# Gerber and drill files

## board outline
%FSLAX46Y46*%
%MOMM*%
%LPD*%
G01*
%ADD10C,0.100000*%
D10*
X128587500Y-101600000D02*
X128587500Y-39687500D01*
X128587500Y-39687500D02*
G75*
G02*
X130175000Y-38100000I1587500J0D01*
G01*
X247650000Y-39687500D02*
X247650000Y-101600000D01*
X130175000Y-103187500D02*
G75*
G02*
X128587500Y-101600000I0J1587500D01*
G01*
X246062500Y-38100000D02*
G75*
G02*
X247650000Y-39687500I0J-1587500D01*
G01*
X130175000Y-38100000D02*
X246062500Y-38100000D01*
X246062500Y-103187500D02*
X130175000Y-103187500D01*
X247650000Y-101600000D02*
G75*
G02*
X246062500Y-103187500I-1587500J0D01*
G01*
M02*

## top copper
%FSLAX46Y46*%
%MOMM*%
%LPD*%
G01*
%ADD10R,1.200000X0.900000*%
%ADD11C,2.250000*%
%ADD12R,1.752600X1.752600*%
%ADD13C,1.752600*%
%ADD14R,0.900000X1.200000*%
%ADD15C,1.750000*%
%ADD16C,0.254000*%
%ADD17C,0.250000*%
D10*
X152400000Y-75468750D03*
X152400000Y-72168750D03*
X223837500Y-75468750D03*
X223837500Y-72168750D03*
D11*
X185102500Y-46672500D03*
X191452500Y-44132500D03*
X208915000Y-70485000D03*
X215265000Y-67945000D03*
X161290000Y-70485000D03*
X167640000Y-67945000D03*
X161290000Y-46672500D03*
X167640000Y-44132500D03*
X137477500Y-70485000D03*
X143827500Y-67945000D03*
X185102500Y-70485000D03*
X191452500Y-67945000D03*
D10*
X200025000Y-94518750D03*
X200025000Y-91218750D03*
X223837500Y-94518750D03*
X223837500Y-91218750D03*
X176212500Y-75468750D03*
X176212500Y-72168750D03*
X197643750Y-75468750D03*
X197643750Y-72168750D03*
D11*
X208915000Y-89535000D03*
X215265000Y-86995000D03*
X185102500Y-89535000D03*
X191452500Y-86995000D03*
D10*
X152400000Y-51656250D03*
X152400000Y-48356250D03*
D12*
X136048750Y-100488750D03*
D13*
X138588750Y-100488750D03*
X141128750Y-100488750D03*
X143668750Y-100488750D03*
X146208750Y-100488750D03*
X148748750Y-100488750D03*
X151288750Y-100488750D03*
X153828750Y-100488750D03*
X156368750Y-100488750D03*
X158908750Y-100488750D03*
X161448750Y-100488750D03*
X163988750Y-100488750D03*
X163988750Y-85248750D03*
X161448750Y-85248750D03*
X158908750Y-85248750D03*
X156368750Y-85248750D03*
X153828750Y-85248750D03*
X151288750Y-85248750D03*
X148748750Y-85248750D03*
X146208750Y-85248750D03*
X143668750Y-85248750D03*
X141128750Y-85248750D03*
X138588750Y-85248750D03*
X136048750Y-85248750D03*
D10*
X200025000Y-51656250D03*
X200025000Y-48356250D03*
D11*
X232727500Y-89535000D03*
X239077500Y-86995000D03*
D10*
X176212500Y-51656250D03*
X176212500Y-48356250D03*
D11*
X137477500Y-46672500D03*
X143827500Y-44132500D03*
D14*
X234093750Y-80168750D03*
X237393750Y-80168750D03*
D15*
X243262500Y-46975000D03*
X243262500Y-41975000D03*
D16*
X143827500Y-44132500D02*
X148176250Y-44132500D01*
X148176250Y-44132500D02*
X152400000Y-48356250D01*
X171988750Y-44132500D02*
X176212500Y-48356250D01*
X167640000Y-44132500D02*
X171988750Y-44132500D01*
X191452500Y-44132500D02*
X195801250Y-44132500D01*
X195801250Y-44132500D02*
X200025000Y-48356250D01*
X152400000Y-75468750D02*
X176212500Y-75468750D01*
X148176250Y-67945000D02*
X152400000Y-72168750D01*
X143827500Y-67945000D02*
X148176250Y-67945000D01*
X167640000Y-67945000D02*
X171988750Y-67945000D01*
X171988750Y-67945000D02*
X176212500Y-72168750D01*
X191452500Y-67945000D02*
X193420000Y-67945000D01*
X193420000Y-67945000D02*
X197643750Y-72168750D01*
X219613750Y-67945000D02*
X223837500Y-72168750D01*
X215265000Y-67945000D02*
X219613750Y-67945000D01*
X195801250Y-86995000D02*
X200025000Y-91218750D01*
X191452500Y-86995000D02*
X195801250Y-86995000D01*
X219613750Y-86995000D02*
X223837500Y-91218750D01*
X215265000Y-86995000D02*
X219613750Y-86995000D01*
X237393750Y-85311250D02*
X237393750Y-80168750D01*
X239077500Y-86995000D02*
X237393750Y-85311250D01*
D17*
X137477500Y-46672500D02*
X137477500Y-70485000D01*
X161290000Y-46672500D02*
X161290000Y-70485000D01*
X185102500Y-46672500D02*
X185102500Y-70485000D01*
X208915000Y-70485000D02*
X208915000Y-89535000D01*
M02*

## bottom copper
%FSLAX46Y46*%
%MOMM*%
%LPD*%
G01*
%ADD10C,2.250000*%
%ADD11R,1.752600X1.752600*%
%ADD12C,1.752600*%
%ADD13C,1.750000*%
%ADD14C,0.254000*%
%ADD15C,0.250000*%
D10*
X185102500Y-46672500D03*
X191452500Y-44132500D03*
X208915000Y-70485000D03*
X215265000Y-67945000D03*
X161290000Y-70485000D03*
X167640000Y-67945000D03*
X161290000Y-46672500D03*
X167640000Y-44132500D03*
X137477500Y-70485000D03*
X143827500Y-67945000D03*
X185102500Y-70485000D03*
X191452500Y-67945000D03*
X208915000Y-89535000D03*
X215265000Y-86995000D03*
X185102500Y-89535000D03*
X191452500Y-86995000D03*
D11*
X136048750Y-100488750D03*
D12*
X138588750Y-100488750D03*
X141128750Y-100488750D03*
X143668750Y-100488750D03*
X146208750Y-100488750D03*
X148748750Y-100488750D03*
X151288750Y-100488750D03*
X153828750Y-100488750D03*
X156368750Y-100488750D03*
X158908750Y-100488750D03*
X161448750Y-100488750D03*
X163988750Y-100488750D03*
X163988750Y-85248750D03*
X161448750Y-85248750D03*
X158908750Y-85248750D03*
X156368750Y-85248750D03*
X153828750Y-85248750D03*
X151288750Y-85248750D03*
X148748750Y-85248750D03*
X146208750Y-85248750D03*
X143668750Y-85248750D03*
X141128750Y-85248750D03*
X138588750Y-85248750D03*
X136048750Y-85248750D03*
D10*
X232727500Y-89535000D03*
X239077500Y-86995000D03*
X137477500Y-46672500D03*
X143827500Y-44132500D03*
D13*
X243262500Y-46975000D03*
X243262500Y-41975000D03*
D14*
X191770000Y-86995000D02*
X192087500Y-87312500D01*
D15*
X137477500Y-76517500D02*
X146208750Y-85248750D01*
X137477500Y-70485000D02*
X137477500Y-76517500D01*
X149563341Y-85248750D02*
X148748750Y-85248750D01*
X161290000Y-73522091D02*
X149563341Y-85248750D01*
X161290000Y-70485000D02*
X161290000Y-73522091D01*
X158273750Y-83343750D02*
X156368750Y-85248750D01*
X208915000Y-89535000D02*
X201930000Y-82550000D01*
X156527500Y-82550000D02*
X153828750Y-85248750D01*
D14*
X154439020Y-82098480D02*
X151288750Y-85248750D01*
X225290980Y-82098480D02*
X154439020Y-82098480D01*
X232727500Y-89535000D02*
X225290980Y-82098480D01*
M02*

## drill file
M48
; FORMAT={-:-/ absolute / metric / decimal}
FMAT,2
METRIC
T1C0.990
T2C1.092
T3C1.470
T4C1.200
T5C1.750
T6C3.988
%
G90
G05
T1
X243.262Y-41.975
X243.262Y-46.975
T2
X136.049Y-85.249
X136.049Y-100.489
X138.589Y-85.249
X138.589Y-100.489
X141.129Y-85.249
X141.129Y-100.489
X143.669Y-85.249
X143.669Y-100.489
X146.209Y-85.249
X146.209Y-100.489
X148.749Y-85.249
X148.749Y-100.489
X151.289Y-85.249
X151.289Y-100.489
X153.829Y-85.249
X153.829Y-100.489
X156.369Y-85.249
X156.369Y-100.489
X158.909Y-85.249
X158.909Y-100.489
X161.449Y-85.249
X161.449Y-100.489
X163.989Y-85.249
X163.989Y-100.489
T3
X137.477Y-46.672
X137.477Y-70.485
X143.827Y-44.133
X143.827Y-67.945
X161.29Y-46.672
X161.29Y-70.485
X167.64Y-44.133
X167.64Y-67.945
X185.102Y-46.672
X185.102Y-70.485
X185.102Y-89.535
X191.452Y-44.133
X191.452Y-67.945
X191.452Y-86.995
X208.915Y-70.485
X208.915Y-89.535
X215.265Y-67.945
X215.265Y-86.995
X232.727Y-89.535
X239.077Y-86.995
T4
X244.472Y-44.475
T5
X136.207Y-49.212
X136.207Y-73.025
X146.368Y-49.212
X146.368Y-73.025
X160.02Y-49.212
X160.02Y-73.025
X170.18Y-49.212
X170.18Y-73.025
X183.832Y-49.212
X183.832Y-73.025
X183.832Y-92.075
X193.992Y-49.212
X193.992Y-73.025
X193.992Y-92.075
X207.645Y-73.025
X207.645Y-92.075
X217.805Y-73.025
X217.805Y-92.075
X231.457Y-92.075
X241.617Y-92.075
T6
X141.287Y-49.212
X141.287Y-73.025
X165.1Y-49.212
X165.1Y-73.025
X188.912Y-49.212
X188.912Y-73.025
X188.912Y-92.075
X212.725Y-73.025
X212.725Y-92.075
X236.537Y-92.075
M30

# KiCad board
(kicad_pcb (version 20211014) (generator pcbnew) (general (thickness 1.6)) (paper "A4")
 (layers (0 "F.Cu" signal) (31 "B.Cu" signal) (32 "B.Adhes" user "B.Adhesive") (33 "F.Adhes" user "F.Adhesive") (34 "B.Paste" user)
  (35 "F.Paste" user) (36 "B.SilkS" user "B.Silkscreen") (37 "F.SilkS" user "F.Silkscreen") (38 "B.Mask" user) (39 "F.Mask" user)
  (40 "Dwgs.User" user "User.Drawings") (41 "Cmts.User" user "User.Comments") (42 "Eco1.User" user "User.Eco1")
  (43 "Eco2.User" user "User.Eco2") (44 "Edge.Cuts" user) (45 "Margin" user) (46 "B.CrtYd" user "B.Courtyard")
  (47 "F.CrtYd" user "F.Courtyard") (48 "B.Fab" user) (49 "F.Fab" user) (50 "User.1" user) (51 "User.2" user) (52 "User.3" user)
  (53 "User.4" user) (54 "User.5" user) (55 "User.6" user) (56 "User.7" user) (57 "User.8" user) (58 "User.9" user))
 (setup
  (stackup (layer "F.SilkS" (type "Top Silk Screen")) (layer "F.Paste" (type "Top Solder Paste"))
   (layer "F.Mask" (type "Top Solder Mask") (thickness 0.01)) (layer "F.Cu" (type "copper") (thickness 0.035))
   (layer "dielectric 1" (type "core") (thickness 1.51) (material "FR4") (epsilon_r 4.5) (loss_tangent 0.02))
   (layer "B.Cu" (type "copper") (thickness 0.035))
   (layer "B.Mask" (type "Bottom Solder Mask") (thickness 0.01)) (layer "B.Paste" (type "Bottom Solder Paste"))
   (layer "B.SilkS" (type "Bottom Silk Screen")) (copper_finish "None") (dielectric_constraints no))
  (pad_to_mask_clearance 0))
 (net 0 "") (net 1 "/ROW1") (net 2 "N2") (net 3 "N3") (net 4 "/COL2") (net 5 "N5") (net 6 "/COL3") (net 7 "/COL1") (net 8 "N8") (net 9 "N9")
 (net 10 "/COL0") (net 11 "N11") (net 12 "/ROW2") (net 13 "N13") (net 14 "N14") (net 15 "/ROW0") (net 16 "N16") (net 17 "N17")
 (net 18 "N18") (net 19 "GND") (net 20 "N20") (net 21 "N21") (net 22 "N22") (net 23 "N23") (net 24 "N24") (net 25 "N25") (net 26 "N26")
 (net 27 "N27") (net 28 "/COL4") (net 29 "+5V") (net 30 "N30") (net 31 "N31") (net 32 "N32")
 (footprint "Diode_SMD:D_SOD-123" (layer "F.Cu") (at 152.4 73.81875 90)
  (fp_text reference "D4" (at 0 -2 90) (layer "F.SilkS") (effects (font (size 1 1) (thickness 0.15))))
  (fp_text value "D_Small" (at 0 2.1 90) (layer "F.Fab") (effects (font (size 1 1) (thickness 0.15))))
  (pad "1" smd rect (at -1.65 0 90) (size 0.9 1.2) (layers "F.Cu" "F.Paste" "F.Mask") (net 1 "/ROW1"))
  (pad "2" smd rect (at 1.65 0 90) (size 0.9 1.2) (layers "F.Cu" "F.Paste" "F.Mask") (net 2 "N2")))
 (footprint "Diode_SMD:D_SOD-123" (layer "F.Cu") (at 223.8375 73.81875 90)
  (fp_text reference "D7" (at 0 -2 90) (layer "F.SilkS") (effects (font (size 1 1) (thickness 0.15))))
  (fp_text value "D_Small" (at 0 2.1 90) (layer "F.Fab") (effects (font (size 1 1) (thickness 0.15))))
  (pad "1" smd rect (at -1.65 0 90) (size 0.9 1.2) (layers "F.Cu" "F.Paste" "F.Mask") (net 1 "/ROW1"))
  (pad "2" smd rect (at 1.65 0 90) (size 0.9 1.2) (layers "F.Cu" "F.Paste" "F.Mask") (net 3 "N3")))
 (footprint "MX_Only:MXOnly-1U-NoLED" (layer "F.Cu") (at 188.9125 49.2125)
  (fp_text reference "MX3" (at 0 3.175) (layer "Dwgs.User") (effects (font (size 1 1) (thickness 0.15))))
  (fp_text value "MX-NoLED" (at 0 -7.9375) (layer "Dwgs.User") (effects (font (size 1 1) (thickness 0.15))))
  (pad "" np_thru_hole circle locked (at 0 0) (size 3.9878 3.9878) (drill 3.9878) (layers *.Cu *.Mask))
  (pad "" np_thru_hole circle locked (at -5.08 0 48.0996) (size 1.75 1.75) (drill 1.75) (layers *.Cu *.Mask))
  (pad "" np_thru_hole circle locked (at 5.08 0 48.0996) (size 1.75 1.75) (drill 1.75) (layers *.Cu *.Mask))
  (pad "1" thru_hole circle locked (at -3.81 -2.54) (size 2.25 2.25) (drill 1.47) (layers *.Cu "B.Mask") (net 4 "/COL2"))
  (pad "2" thru_hole circle locked (at 2.54 -5.08) (size 2.25 2.25) (drill 1.47) (layers *.Cu "B.Mask") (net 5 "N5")))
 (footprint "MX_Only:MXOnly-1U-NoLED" (layer "F.Cu") (at 212.725 73.025)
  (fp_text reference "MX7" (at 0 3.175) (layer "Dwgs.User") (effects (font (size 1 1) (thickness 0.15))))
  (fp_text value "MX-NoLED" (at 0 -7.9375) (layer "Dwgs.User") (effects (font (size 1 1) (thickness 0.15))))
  (pad "" np_thru_hole circle locked (at 5.08 0 48.0996) (size 1.75 1.75) (drill 1.75) (layers *.Cu *.Mask))
  (pad "" np_thru_hole circle locked (at 0 0) (size 3.9878 3.9878) (drill 3.9878) (layers *.Cu *.Mask))
  (pad "" np_thru_hole circle locked (at -5.08 0 48.0996) (size 1.75 1.75) (drill 1.75) (layers *.Cu *.Mask))
  (pad "1" thru_hole circle locked (at -3.81 -2.54) (size 2.25 2.25) (drill 1.47) (layers *.Cu "B.Mask") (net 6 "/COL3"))
  (pad "2" thru_hole circle locked (at 2.54 -5.08) (size 2.25 2.25) (drill 1.47) (layers *.Cu "B.Mask") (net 3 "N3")))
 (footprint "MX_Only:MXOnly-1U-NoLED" (layer "F.Cu") (at 165.1 73.025)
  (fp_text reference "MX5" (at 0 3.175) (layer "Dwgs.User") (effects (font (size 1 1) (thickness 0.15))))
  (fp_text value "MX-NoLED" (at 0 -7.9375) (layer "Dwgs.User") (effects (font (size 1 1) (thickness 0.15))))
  (pad "" np_thru_hole circle locked (at 5.08 0 48.0996) (size 1.75 1.75) (drill 1.75) (layers *.Cu *.Mask))
  (pad "" np_thru_hole circle locked (at -5.08 0 48.0996) (size 1.75 1.75) (drill 1.75) (layers *.Cu *.Mask))
  (pad "" np_thru_hole circle locked (at 0 0) (size 3.9878 3.9878) (drill 3.9878) (layers *.Cu *.Mask))
  (pad "1" thru_hole circle locked (at -3.81 -2.54) (size 2.25 2.25) (drill 1.47) (layers *.Cu "B.Mask") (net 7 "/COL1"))
  (pad "2" thru_hole circle locked (at 2.54 -5.08) (size 2.25 2.25) (drill 1.47) (layers *.Cu "B.Mask") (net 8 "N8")))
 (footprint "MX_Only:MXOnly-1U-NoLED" (layer "F.Cu") (at 165.1 49.2125)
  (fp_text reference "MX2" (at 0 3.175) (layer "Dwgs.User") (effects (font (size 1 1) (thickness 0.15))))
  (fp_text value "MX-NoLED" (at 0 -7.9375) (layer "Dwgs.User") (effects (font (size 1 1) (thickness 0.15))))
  (pad "" np_thru_hole circle locked (at 5.08 0 48.0996) (size 1.75 1.75) (drill 1.75) (layers *.Cu *.Mask))
  (pad "" np_thru_hole circle locked (at 0 0) (size 3.9878 3.9878) (drill 3.9878) (layers *.Cu *.Mask))
  (pad "" np_thru_hole circle locked (at -5.08 0 48.0996) (size 1.75 1.75) (drill 1.75) (layers *.Cu *.Mask))
  (pad "1" thru_hole circle locked (at -3.81 -2.54) (size 2.25 2.25) (drill 1.47) (layers *.Cu "B.Mask") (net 7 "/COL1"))
  (pad "2" thru_hole circle locked (at 2.54 -5.08) (size 2.25 2.25) (drill 1.47) (layers *.Cu "B.Mask") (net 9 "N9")))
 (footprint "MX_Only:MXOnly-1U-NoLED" (layer "F.Cu") (at 141.2875 73.025)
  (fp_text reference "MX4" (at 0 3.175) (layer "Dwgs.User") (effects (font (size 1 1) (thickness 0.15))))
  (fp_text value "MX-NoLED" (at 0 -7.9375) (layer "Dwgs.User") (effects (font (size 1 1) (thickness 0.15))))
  (pad "" np_thru_hole circle locked (at 0 0) (size 3.9878 3.9878) (drill 3.9878) (layers *.Cu *.Mask))
  (pad "" np_thru_hole circle locked (at -5.08 0 48.0996) (size 1.75 1.75) (drill 1.75) (layers *.Cu *.Mask))
  (pad "" np_thru_hole circle locked (at 5.08 0 48.0996) (size 1.75 1.75) (drill 1.75) (layers *.Cu *.Mask))
  (pad "1" thru_hole circle locked (at -3.81 -2.54) (size 2.25 2.25) (drill 1.47) (layers *.Cu "B.Mask") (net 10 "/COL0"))
  (pad "2" thru_hole circle locked (at 2.54 -5.08) (size 2.25 2.25) (drill 1.47) (layers *.Cu "B.Mask") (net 2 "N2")))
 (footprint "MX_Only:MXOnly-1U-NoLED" (layer "F.Cu") (at 188.9125 73.025)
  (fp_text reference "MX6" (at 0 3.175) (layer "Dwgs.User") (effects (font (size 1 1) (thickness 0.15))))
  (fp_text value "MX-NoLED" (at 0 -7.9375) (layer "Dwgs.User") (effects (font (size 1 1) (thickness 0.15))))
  (pad "" np_thru_hole circle locked (at -5.08 0 48.0996) (size 1.75 1.75) (drill 1.75) (layers *.Cu *.Mask))
  (pad "" np_thru_hole circle locked (at 5.08 0 48.0996) (size 1.75 1.75) (drill 1.75) (layers *.Cu *.Mask))
  (pad "" np_thru_hole circle locked (at 0 0) (size 3.9878 3.9878) (drill 3.9878) (layers *.Cu *.Mask))
  (pad "1" thru_hole circle locked (at -3.81 -2.54) (size 2.25 2.25) (drill 1.47) (layers *.Cu "B.Mask") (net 4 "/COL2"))
  (pad "2" thru_hole circle locked (at 2.54 -5.08) (size 2.25 2.25) (drill 1.47) (layers *.Cu "B.Mask") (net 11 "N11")))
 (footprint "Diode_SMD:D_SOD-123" (layer "F.Cu") (at 200.025 92.86875 90)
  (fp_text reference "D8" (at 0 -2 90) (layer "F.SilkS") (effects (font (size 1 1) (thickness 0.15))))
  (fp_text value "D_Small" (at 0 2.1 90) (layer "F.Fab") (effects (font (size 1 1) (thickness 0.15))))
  (pad "1" smd rect (at -1.65 0 90) (size 0.9 1.2) (layers "F.Cu" "F.Paste" "F.Mask") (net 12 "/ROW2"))
  (pad "2" smd rect (at 1.65 0 90) (size 0.9 1.2) (layers "F.Cu" "F.Paste" "F.Mask") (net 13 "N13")))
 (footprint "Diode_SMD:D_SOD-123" (layer "F.Cu") (at 223.8375 92.86875 90)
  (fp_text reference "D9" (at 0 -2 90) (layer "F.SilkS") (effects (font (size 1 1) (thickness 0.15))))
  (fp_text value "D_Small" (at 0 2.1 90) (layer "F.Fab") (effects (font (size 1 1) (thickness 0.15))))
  (pad "1" smd rect (at -1.65 0 90) (size 0.9 1.2) (layers "F.Cu" "F.Paste" "F.Mask") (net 12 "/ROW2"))
  (pad "2" smd rect (at 1.65 0 90) (size 0.9 1.2) (layers "F.Cu" "F.Paste" "F.Mask") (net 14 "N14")))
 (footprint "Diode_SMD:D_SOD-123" (layer "F.Cu") (at 176.2125 73.81875 90)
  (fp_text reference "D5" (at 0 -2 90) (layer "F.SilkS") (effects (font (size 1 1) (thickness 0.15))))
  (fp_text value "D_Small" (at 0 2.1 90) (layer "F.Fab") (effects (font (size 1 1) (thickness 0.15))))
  (pad "1" smd rect (at -1.65 0 90) (size 0.9 1.2) (layers "F.Cu" "F.Paste" "F.Mask") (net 1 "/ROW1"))
  (pad "2" smd rect (at 1.65 0 90) (size 0.9 1.2) (layers "F.Cu" "F.Paste" "F.Mask") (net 8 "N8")))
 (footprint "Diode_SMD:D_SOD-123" (layer "F.Cu") (at 197.64375 73.81875 90)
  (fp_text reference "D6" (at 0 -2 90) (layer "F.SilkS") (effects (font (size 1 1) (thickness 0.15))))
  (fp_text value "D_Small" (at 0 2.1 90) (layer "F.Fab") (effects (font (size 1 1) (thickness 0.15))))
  (pad "1" smd rect (at -1.65 0 90) (size 0.9 1.2) (layers "F.Cu" "F.Paste" "F.Mask") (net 1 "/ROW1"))
  (pad "2" smd rect (at 1.65 0 90) (size 0.9 1.2) (layers "F.Cu" "F.Paste" "F.Mask") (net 11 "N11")))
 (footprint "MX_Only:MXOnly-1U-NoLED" (layer "F.Cu") (at 212.725 92.075)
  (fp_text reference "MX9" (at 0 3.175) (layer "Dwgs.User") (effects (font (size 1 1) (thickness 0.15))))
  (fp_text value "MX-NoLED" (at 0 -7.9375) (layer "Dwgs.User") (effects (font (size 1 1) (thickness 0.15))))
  (pad "" np_thru_hole circle locked (at 0 0) (size 3.9878 3.9878) (drill 3.9878) (layers *.Cu *.Mask))
  (pad "" np_thru_hole circle locked (at 5.08 0 48.0996) (size 1.75 1.75) (drill 1.75) (layers *.Cu *.Mask))
  (pad "" np_thru_hole circle locked (at -5.08 0 48.0996) (size 1.75 1.75) (drill 1.75) (layers *.Cu *.Mask))
  (pad "1" thru_hole circle locked (at -3.81 -2.54) (size 2.25 2.25) (drill 1.47) (layers *.Cu "B.Mask") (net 6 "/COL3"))
  (pad "2" thru_hole circle locked (at 2.54 -5.08) (size 2.25 2.25) (drill 1.47) (layers *.Cu "B.Mask") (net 14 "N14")))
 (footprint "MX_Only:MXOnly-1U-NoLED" (layer "F.Cu") (at 188.9125 92.075)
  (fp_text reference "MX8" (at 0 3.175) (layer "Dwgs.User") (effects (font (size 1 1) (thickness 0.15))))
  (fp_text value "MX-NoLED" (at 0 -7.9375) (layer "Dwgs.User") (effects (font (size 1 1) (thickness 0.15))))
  (pad "" np_thru_hole circle locked (at 5.08 0 48.0996) (size 1.75 1.75) (drill 1.75) (layers *.Cu *.Mask))
  (pad "" np_thru_hole circle locked (at 0 0) (size 3.9878 3.9878) (drill 3.9878) (layers *.Cu *.Mask))
  (pad "" np_thru_hole circle locked (at -5.08 0 48.0996) (size 1.75 1.75) (drill 1.75) (layers *.Cu *.Mask))
  (pad "1" thru_hole circle locked (at -3.81 -2.54) (size 2.25 2.25) (drill 1.47) (layers *.Cu "B.Mask") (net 4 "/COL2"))
  (pad "2" thru_hole circle locked (at 2.54 -5.08) (size 2.25 2.25) (drill 1.47) (layers *.Cu "B.Mask") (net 13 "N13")))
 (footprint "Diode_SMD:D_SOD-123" (layer "F.Cu") (at 152.4 50.00625 90)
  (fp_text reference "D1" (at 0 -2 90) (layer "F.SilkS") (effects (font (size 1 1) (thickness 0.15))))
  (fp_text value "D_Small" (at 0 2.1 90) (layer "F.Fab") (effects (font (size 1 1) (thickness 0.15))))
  (pad "1" smd rect (at -1.65 0 90) (size 0.9 1.2) (layers "F.Cu" "F.Paste" "F.Mask") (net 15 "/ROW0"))
  (pad "2" smd rect (at 1.65 0 90) (size 0.9 1.2) (layers "F.Cu" "F.Paste" "F.Mask") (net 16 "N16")))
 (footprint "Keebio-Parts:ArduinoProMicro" (layer "F.Cu") (at 150.01875 92.86875)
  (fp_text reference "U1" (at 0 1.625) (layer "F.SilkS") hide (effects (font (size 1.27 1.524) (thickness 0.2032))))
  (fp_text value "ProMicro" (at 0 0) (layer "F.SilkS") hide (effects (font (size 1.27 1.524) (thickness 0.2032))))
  (pad "1" thru_hole rect locked (at -13.97 7.62) (size 1.7526 1.7526) (drill 1.0922) (layers *.Cu *.SilkS *.Mask) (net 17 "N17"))
  (pad "2" thru_hole circle locked (at -11.43 7.62) (size 1.7526 1.7526) (drill 1.0922) (layers *.Cu *.SilkS *.Mask) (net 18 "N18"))
  (pad "3" thru_hole circle locked (at -8.89 7.62) (size 1.7526 1.7526) (drill 1.0922) (layers *.Cu *.SilkS *.Mask) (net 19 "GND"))
  (pad "4" thru_hole circle locked (at -6.35 7.62) (size 1.7526 1.7526) (drill 1.0922) (layers *.Cu *.SilkS *.Mask) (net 19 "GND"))
  (pad "5" thru_hole circle locked (at -3.81 7.62) (size 1.7526 1.7526) (drill 1.0922) (layers *.Cu *.SilkS *.Mask) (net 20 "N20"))
  (pad "6" thru_hole circle locked (at -1.27 7.62) (size 1.7526 1.7526) (drill 1.0922) (layers *.Cu *.SilkS *.Mask) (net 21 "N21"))
  (pad "7" thru_hole circle locked (at 1.27 7.62) (size 1.7526 1.7526) (drill 1.0922) (layers *.Cu *.SilkS *.Mask) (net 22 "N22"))
  (pad "8" thru_hole circle locked (at 3.81 7.62) (size 1.7526 1.7526) (drill 1.0922) (layers *.Cu *.SilkS *.Mask) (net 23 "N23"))
  (pad "9" thru_hole circle locked (at 6.35 7.62) (size 1.7526 1.7526) (drill 1.0922) (layers *.Cu *.SilkS *.Mask) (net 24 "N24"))
  (pad "10" thru_hole circle locked (at 8.89 7.62) (size 1.7526 1.7526) (drill 1.0922) (layers *.Cu *.SilkS *.Mask) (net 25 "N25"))
  (pad "11" thru_hole circle locked (at 11.43 7.62) (size 1.7526 1.7526) (drill 1.0922) (layers *.Cu *.SilkS *.Mask) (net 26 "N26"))
  (pad "12" thru_hole circle locked (at 13.97 7.62) (size 1.7526 1.7526) (drill 1.0922) (layers *.Cu *.SilkS *.Mask) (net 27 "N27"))
  (pad "13" thru_hole circle locked (at 13.97 -7.62) (size 1.7526 1.7526) (drill 1.0922) (layers *.Cu *.SilkS *.Mask) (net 12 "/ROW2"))
  (pad "14" thru_hole circle locked (at 11.43 -7.62) (size 1.7526 1.7526) (drill 1.0922) (layers *.Cu *.SilkS *.Mask) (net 1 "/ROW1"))
  (pad "15" thru_hole circle locked (at 8.89 -7.62) (size 1.7526 1.7526) (drill 1.0922) (layers *.Cu *.SilkS *.Mask) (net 15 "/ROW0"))
  (pad "16" thru_hole circle locked (at 6.35 -7.62) (size 1.7526 1.7526) (drill 1.0922) (layers *.Cu *.SilkS *.Mask) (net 4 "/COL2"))
  (pad "17" thru_hole circle locked (at 3.81 -7.62) (size 1.7526 1.7526) (drill 1.0922) (layers *.Cu *.SilkS *.Mask) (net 6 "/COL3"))
  (pad "18" thru_hole circle locked (at 1.27 -7.62) (size 1.7526 1.7526) (drill 1.0922) (layers *.Cu *.SilkS *.Mask) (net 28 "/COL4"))
  (pad "19" thru_hole circle locked (at -1.27 -7.62) (size 1.7526 1.7526) (drill 1.0922) (layers *.Cu *.SilkS *.Mask) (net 7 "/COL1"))
  (pad "20" thru_hole circle locked (at -3.81 -7.62) (size 1.7526 1.7526) (drill 1.0922) (layers *.Cu *.SilkS *.Mask) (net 10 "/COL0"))
  (pad "21" thru_hole circle locked (at -6.35 -7.62) (size 1.7526 1.7526) (drill 1.0922) (layers *.Cu *.SilkS *.Mask) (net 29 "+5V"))
  (pad "22" thru_hole circle locked (at -8.89 -7.62) (size 1.7526 1.7526) (drill 1.0922) (layers *.Cu *.SilkS *.Mask) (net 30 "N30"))
  (pad "23" thru_hole circle locked (at -11.43 -7.62) (size 1.7526 1.7526) (drill 1.0922) (layers *.Cu *.SilkS *.Mask) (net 19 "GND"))
  (pad "24" thru_hole circle locked (at -13.97 -7.62) (size 1.7526 1.7526) (drill 1.0922) (layers *.Cu *.SilkS *.Mask) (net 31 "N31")))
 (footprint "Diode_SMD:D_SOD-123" (layer "F.Cu") (at 200.025 50.00625 90)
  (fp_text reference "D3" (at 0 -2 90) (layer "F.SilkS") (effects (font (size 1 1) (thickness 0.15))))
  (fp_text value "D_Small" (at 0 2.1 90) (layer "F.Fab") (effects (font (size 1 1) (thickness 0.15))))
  (pad "1" smd rect (at -1.65 0 90) (size 0.9 1.2) (layers "F.Cu" "F.Paste" "F.Mask") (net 15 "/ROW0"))
  (pad "2" smd rect (at 1.65 0 90) (size 0.9 1.2) (layers "F.Cu" "F.Paste" "F.Mask") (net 5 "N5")))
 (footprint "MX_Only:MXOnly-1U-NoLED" (layer "F.Cu") (at 236.5375 92.075)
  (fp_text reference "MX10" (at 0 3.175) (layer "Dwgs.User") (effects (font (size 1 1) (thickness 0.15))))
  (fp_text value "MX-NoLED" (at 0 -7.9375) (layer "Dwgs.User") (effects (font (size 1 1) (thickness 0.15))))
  (pad "" np_thru_hole circle locked (at 0 0) (size 3.9878 3.9878) (drill 3.9878) (layers *.Cu *.Mask))
  (pad "" np_thru_hole circle locked (at 5.08 0 48.0996) (size 1.75 1.75) (drill 1.75) (layers *.Cu *.Mask))
  (pad "" np_thru_hole circle locked (at -5.08 0 48.0996) (size 1.75 1.75) (drill 1.75) (layers *.Cu *.Mask))
  (pad "1" thru_hole circle locked (at -3.81 -2.54) (size 2.25 2.25) (drill 1.47) (layers *.Cu "B.Mask") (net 28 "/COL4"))
  (pad "2" thru_hole circle locked (at 2.54 -5.08) (size 2.25 2.25) (drill 1.47) (layers *.Cu "B.Mask") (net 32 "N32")))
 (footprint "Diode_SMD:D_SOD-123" (layer "F.Cu") (at 176.2125 50.00625 90)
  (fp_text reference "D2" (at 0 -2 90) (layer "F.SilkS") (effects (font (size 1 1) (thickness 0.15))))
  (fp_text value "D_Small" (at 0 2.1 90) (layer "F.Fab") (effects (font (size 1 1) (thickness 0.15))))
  (pad "1" smd rect (at -1.65 0 90) (size 0.9 1.2) (layers "F.Cu" "F.Paste" "F.Mask") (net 15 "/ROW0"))
  (pad "2" smd rect (at 1.65 0 90) (size 0.9 1.2) (layers "F.Cu" "F.Paste" "F.Mask") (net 9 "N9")))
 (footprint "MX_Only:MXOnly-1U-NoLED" (layer "F.Cu") (at 141.2875 49.2125)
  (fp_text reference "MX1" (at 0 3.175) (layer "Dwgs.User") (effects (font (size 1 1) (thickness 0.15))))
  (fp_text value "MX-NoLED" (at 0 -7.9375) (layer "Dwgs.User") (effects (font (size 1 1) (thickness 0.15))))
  (pad "" np_thru_hole circle locked (at 0 0) (size 3.9878 3.9878) (drill 3.9878) (layers *.Cu *.Mask))
  (pad "" np_thru_hole circle locked (at -5.08 0 48.0996) (size 1.75 1.75) (drill 1.75) (layers *.Cu *.Mask))
  (pad "" np_thru_hole circle locked (at 5.08 0 48.0996) (size 1.75 1.75) (drill 1.75) (layers *.Cu *.Mask))
  (pad "1" thru_hole circle locked (at -3.81 -2.54) (size 2.25 2.25) (drill 1.47) (layers *.Cu "B.Mask") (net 10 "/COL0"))
  (pad "2" thru_hole circle locked (at 2.54 -5.08) (size 2.25 2.25) (drill 1.47) (layers *.Cu "B.Mask") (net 16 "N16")))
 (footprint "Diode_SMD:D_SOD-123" (layer "F.Cu") (at 235.74375 80.16875)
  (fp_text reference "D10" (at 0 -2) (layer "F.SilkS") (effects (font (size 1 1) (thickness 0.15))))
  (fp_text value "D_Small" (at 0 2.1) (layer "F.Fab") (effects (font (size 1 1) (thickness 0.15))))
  (pad "1" smd rect (at -1.65 0) (size 0.9 1.2) (layers "F.Cu" "F.Paste" "F.Mask") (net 12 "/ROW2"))
  (pad "2" smd rect (at 1.65 0) (size 0.9 1.2) (layers "F.Cu" "F.Paste" "F.Mask") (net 32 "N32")))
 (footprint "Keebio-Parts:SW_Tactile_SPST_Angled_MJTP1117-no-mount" (layer "B.Cu") (at 243.2625 46.975 90)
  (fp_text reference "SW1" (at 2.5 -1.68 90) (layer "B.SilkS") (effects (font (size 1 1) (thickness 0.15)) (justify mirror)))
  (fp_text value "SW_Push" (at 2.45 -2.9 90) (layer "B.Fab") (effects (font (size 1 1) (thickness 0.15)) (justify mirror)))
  (pad "" np_thru_hole circle locked (at 2.5 1.21 90) (size 1.2 1.2) (drill 1.2) (layers *.Cu *.Mask))
  (pad "1" thru_hole circle locked (at 0 0 90) (size 1.75 1.75) (drill 0.99) (layers *.Cu *.Mask) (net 30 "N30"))
  (pad "2" thru_hole circle locked (at 5 0 90) (size 1.75 1.75) (drill 0.99) (layers *.Cu *.Mask) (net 19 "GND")))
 (gr_line (start 128.5875 101.6) (end 128.5875 39.6875) (layer "Edge.Cuts") (width 0.1))
 (gr_arc (start 128.5875 39.6875) (mid 129.052468 38.564968) (end 130.175 38.1) (layer "Edge.Cuts") (width 0.1))
 (gr_line (start 247.65 39.6875) (end 247.65 101.6) (layer "Edge.Cuts") (width 0.1))
 (gr_arc (start 130.175 103.1875) (mid 129.052468 102.722532) (end 128.5875 101.6) (layer "Edge.Cuts") (width 0.1))
 (gr_arc (start 246.0625 38.1) (mid 247.185032 38.564968) (end 247.65 39.6875) (layer "Edge.Cuts") (width 0.1))
 (gr_line (start 130.175 38.1) (end 246.0625 38.1) (layer "Edge.Cuts") (width 0.1))
 (gr_line (start 246.0625 103.1875) (end 130.175 103.1875) (layer "Edge.Cuts") (width 0.1))
 (gr_arc (start 247.65 101.6) (mid 247.185032 102.722532) (end 246.0625 103.1875) (layer "Edge.Cuts") (width 0.1))
 (segment (start 143.8275 44.1325) (end 148.17625 44.1325) (width 0.254) (layer "F.Cu") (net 16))
 (segment (start 148.17625 44.1325) (end 152.4 48.35625) (width 0.254) (layer "F.Cu") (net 16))
 (segment (start 171.98875 44.1325) (end 176.2125 48.35625) (width 0.254) (layer "F.Cu") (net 9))
 (segment (start 167.64 44.1325) (end 171.98875 44.1325) (width 0.254) (layer "F.Cu") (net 9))
 (segment (start 191.4525 44.1325) (end 195.80125 44.1325) (width 0.254) (layer "F.Cu") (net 5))
 (segment (start 195.80125 44.1325) (end 200.025 48.35625) (width 0.254) (layer "F.Cu") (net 5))
 (segment (start 152.4 75.46875) (end 176.2125 75.46875) (width 0.254) (layer "F.Cu") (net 1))
 (segment (start 148.17625 67.945) (end 152.4 72.16875) (width 0.254) (layer "F.Cu") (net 2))
 (segment (start 143.8275 67.945) (end 148.17625 67.945) (width 0.254) (layer "F.Cu") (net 2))
 (segment (start 167.64 67.945) (end 171.98875 67.945) (width 0.254) (layer "F.Cu") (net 8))
 (segment (start 171.98875 67.945) (end 176.2125 72.16875) (width 0.254) (layer "F.Cu") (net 8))
 (segment (start 191.4525 67.945) (end 193.42 67.945) (width 0.254) (layer "F.Cu") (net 11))
 (segment (start 193.42 67.945) (end 197.64375 72.16875) (width 0.254) (layer "F.Cu") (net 11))
 (segment (start 219.61375 67.945) (end 223.8375 72.16875) (width 0.254) (layer "F.Cu") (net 3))
 (segment (start 215.265 67.945) (end 219.61375 67.945) (width 0.254) (layer "F.Cu") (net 3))
 (segment (start 195.80125 86.995) (end 200.025 91.21875) (width 0.254) (layer "F.Cu") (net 13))
 (segment (start 191.4525 86.995) (end 195.80125 86.995) (width 0.254) (layer "F.Cu") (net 13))
 (segment (start 191.77 86.995) (end 192.0875 87.3125) (width 0.254) (layer "B.Cu") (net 13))
 (segment (start 219.61375 86.995) (end 223.8375 91.21875) (width 0.254) (layer "F.Cu") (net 14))
 (segment (start 215.265 86.995) (end 219.61375 86.995) (width 0.254) (layer "F.Cu") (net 14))
 (segment (start 237.39375 85.31125) (end 237.39375 80.16875) (width 0.254) (layer "F.Cu") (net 32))
 (segment (start 239.0775 86.995) (end 237.39375 85.31125) (width 0.254) (layer "F.Cu") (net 32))
 (segment (start 137.4775 46.6725) (end 137.4775 70.485) (width 0.25) (layer "F.Cu") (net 10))
 (segment (start 137.4775 76.5175) (end 146.20875 85.24875) (width 0.25) (layer "B.Cu") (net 10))
 (segment (start 137.4775 70.485) (end 137.4775 76.5175) (width 0.25) (layer "B.Cu") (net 10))
 (segment (start 161.29 46.6725) (end 161.29 70.485) (width 0.25) (layer "F.Cu") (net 7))
 (segment (start 149.563341 85.24875) (end 148.74875 85.24875) (width 0.25) (layer "B.Cu") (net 7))
 (segment (start 161.29 73.522091) (end 149.563341 85.24875) (width 0.25) (layer "B.Cu") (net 7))
 (segment (start 161.29 70.485) (end 161.29 73.522091) (width 0.25) (layer "B.Cu") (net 7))
 (segment (start 185.1025 46.6725) (end 185.1025 70.485) (width 0.25) (layer "F.Cu") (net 4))
 (segment (start 158.27375 83.34375) (end 156.36875 85.24875) (width 0.25) (layer "B.Cu") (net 4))
 (segment (start 208.915 70.485) (end 208.915 89.535) (width 0.25) (layer "F.Cu") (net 6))
 (segment (start 208.915 89.535) (end 201.93 82.55) (width 0.25) (layer "B.Cu") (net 6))
 (segment (start 156.5275 82.55) (end 153.82875 85.24875) (width 0.25) (layer "B.Cu") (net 6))
 (segment (start 154.43902 82.09848) (end 151.28875 85.24875) (width 0.254) (layer "B.Cu") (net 28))
 (segment (start 225.29098 82.09848) (end 154.43902 82.09848) (width 0.254) (layer "B.Cu") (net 28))
 (segment (start 232.7275 89.535) (end 225.29098 82.09848) (width 0.254) (layer "B.Cu") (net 28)))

